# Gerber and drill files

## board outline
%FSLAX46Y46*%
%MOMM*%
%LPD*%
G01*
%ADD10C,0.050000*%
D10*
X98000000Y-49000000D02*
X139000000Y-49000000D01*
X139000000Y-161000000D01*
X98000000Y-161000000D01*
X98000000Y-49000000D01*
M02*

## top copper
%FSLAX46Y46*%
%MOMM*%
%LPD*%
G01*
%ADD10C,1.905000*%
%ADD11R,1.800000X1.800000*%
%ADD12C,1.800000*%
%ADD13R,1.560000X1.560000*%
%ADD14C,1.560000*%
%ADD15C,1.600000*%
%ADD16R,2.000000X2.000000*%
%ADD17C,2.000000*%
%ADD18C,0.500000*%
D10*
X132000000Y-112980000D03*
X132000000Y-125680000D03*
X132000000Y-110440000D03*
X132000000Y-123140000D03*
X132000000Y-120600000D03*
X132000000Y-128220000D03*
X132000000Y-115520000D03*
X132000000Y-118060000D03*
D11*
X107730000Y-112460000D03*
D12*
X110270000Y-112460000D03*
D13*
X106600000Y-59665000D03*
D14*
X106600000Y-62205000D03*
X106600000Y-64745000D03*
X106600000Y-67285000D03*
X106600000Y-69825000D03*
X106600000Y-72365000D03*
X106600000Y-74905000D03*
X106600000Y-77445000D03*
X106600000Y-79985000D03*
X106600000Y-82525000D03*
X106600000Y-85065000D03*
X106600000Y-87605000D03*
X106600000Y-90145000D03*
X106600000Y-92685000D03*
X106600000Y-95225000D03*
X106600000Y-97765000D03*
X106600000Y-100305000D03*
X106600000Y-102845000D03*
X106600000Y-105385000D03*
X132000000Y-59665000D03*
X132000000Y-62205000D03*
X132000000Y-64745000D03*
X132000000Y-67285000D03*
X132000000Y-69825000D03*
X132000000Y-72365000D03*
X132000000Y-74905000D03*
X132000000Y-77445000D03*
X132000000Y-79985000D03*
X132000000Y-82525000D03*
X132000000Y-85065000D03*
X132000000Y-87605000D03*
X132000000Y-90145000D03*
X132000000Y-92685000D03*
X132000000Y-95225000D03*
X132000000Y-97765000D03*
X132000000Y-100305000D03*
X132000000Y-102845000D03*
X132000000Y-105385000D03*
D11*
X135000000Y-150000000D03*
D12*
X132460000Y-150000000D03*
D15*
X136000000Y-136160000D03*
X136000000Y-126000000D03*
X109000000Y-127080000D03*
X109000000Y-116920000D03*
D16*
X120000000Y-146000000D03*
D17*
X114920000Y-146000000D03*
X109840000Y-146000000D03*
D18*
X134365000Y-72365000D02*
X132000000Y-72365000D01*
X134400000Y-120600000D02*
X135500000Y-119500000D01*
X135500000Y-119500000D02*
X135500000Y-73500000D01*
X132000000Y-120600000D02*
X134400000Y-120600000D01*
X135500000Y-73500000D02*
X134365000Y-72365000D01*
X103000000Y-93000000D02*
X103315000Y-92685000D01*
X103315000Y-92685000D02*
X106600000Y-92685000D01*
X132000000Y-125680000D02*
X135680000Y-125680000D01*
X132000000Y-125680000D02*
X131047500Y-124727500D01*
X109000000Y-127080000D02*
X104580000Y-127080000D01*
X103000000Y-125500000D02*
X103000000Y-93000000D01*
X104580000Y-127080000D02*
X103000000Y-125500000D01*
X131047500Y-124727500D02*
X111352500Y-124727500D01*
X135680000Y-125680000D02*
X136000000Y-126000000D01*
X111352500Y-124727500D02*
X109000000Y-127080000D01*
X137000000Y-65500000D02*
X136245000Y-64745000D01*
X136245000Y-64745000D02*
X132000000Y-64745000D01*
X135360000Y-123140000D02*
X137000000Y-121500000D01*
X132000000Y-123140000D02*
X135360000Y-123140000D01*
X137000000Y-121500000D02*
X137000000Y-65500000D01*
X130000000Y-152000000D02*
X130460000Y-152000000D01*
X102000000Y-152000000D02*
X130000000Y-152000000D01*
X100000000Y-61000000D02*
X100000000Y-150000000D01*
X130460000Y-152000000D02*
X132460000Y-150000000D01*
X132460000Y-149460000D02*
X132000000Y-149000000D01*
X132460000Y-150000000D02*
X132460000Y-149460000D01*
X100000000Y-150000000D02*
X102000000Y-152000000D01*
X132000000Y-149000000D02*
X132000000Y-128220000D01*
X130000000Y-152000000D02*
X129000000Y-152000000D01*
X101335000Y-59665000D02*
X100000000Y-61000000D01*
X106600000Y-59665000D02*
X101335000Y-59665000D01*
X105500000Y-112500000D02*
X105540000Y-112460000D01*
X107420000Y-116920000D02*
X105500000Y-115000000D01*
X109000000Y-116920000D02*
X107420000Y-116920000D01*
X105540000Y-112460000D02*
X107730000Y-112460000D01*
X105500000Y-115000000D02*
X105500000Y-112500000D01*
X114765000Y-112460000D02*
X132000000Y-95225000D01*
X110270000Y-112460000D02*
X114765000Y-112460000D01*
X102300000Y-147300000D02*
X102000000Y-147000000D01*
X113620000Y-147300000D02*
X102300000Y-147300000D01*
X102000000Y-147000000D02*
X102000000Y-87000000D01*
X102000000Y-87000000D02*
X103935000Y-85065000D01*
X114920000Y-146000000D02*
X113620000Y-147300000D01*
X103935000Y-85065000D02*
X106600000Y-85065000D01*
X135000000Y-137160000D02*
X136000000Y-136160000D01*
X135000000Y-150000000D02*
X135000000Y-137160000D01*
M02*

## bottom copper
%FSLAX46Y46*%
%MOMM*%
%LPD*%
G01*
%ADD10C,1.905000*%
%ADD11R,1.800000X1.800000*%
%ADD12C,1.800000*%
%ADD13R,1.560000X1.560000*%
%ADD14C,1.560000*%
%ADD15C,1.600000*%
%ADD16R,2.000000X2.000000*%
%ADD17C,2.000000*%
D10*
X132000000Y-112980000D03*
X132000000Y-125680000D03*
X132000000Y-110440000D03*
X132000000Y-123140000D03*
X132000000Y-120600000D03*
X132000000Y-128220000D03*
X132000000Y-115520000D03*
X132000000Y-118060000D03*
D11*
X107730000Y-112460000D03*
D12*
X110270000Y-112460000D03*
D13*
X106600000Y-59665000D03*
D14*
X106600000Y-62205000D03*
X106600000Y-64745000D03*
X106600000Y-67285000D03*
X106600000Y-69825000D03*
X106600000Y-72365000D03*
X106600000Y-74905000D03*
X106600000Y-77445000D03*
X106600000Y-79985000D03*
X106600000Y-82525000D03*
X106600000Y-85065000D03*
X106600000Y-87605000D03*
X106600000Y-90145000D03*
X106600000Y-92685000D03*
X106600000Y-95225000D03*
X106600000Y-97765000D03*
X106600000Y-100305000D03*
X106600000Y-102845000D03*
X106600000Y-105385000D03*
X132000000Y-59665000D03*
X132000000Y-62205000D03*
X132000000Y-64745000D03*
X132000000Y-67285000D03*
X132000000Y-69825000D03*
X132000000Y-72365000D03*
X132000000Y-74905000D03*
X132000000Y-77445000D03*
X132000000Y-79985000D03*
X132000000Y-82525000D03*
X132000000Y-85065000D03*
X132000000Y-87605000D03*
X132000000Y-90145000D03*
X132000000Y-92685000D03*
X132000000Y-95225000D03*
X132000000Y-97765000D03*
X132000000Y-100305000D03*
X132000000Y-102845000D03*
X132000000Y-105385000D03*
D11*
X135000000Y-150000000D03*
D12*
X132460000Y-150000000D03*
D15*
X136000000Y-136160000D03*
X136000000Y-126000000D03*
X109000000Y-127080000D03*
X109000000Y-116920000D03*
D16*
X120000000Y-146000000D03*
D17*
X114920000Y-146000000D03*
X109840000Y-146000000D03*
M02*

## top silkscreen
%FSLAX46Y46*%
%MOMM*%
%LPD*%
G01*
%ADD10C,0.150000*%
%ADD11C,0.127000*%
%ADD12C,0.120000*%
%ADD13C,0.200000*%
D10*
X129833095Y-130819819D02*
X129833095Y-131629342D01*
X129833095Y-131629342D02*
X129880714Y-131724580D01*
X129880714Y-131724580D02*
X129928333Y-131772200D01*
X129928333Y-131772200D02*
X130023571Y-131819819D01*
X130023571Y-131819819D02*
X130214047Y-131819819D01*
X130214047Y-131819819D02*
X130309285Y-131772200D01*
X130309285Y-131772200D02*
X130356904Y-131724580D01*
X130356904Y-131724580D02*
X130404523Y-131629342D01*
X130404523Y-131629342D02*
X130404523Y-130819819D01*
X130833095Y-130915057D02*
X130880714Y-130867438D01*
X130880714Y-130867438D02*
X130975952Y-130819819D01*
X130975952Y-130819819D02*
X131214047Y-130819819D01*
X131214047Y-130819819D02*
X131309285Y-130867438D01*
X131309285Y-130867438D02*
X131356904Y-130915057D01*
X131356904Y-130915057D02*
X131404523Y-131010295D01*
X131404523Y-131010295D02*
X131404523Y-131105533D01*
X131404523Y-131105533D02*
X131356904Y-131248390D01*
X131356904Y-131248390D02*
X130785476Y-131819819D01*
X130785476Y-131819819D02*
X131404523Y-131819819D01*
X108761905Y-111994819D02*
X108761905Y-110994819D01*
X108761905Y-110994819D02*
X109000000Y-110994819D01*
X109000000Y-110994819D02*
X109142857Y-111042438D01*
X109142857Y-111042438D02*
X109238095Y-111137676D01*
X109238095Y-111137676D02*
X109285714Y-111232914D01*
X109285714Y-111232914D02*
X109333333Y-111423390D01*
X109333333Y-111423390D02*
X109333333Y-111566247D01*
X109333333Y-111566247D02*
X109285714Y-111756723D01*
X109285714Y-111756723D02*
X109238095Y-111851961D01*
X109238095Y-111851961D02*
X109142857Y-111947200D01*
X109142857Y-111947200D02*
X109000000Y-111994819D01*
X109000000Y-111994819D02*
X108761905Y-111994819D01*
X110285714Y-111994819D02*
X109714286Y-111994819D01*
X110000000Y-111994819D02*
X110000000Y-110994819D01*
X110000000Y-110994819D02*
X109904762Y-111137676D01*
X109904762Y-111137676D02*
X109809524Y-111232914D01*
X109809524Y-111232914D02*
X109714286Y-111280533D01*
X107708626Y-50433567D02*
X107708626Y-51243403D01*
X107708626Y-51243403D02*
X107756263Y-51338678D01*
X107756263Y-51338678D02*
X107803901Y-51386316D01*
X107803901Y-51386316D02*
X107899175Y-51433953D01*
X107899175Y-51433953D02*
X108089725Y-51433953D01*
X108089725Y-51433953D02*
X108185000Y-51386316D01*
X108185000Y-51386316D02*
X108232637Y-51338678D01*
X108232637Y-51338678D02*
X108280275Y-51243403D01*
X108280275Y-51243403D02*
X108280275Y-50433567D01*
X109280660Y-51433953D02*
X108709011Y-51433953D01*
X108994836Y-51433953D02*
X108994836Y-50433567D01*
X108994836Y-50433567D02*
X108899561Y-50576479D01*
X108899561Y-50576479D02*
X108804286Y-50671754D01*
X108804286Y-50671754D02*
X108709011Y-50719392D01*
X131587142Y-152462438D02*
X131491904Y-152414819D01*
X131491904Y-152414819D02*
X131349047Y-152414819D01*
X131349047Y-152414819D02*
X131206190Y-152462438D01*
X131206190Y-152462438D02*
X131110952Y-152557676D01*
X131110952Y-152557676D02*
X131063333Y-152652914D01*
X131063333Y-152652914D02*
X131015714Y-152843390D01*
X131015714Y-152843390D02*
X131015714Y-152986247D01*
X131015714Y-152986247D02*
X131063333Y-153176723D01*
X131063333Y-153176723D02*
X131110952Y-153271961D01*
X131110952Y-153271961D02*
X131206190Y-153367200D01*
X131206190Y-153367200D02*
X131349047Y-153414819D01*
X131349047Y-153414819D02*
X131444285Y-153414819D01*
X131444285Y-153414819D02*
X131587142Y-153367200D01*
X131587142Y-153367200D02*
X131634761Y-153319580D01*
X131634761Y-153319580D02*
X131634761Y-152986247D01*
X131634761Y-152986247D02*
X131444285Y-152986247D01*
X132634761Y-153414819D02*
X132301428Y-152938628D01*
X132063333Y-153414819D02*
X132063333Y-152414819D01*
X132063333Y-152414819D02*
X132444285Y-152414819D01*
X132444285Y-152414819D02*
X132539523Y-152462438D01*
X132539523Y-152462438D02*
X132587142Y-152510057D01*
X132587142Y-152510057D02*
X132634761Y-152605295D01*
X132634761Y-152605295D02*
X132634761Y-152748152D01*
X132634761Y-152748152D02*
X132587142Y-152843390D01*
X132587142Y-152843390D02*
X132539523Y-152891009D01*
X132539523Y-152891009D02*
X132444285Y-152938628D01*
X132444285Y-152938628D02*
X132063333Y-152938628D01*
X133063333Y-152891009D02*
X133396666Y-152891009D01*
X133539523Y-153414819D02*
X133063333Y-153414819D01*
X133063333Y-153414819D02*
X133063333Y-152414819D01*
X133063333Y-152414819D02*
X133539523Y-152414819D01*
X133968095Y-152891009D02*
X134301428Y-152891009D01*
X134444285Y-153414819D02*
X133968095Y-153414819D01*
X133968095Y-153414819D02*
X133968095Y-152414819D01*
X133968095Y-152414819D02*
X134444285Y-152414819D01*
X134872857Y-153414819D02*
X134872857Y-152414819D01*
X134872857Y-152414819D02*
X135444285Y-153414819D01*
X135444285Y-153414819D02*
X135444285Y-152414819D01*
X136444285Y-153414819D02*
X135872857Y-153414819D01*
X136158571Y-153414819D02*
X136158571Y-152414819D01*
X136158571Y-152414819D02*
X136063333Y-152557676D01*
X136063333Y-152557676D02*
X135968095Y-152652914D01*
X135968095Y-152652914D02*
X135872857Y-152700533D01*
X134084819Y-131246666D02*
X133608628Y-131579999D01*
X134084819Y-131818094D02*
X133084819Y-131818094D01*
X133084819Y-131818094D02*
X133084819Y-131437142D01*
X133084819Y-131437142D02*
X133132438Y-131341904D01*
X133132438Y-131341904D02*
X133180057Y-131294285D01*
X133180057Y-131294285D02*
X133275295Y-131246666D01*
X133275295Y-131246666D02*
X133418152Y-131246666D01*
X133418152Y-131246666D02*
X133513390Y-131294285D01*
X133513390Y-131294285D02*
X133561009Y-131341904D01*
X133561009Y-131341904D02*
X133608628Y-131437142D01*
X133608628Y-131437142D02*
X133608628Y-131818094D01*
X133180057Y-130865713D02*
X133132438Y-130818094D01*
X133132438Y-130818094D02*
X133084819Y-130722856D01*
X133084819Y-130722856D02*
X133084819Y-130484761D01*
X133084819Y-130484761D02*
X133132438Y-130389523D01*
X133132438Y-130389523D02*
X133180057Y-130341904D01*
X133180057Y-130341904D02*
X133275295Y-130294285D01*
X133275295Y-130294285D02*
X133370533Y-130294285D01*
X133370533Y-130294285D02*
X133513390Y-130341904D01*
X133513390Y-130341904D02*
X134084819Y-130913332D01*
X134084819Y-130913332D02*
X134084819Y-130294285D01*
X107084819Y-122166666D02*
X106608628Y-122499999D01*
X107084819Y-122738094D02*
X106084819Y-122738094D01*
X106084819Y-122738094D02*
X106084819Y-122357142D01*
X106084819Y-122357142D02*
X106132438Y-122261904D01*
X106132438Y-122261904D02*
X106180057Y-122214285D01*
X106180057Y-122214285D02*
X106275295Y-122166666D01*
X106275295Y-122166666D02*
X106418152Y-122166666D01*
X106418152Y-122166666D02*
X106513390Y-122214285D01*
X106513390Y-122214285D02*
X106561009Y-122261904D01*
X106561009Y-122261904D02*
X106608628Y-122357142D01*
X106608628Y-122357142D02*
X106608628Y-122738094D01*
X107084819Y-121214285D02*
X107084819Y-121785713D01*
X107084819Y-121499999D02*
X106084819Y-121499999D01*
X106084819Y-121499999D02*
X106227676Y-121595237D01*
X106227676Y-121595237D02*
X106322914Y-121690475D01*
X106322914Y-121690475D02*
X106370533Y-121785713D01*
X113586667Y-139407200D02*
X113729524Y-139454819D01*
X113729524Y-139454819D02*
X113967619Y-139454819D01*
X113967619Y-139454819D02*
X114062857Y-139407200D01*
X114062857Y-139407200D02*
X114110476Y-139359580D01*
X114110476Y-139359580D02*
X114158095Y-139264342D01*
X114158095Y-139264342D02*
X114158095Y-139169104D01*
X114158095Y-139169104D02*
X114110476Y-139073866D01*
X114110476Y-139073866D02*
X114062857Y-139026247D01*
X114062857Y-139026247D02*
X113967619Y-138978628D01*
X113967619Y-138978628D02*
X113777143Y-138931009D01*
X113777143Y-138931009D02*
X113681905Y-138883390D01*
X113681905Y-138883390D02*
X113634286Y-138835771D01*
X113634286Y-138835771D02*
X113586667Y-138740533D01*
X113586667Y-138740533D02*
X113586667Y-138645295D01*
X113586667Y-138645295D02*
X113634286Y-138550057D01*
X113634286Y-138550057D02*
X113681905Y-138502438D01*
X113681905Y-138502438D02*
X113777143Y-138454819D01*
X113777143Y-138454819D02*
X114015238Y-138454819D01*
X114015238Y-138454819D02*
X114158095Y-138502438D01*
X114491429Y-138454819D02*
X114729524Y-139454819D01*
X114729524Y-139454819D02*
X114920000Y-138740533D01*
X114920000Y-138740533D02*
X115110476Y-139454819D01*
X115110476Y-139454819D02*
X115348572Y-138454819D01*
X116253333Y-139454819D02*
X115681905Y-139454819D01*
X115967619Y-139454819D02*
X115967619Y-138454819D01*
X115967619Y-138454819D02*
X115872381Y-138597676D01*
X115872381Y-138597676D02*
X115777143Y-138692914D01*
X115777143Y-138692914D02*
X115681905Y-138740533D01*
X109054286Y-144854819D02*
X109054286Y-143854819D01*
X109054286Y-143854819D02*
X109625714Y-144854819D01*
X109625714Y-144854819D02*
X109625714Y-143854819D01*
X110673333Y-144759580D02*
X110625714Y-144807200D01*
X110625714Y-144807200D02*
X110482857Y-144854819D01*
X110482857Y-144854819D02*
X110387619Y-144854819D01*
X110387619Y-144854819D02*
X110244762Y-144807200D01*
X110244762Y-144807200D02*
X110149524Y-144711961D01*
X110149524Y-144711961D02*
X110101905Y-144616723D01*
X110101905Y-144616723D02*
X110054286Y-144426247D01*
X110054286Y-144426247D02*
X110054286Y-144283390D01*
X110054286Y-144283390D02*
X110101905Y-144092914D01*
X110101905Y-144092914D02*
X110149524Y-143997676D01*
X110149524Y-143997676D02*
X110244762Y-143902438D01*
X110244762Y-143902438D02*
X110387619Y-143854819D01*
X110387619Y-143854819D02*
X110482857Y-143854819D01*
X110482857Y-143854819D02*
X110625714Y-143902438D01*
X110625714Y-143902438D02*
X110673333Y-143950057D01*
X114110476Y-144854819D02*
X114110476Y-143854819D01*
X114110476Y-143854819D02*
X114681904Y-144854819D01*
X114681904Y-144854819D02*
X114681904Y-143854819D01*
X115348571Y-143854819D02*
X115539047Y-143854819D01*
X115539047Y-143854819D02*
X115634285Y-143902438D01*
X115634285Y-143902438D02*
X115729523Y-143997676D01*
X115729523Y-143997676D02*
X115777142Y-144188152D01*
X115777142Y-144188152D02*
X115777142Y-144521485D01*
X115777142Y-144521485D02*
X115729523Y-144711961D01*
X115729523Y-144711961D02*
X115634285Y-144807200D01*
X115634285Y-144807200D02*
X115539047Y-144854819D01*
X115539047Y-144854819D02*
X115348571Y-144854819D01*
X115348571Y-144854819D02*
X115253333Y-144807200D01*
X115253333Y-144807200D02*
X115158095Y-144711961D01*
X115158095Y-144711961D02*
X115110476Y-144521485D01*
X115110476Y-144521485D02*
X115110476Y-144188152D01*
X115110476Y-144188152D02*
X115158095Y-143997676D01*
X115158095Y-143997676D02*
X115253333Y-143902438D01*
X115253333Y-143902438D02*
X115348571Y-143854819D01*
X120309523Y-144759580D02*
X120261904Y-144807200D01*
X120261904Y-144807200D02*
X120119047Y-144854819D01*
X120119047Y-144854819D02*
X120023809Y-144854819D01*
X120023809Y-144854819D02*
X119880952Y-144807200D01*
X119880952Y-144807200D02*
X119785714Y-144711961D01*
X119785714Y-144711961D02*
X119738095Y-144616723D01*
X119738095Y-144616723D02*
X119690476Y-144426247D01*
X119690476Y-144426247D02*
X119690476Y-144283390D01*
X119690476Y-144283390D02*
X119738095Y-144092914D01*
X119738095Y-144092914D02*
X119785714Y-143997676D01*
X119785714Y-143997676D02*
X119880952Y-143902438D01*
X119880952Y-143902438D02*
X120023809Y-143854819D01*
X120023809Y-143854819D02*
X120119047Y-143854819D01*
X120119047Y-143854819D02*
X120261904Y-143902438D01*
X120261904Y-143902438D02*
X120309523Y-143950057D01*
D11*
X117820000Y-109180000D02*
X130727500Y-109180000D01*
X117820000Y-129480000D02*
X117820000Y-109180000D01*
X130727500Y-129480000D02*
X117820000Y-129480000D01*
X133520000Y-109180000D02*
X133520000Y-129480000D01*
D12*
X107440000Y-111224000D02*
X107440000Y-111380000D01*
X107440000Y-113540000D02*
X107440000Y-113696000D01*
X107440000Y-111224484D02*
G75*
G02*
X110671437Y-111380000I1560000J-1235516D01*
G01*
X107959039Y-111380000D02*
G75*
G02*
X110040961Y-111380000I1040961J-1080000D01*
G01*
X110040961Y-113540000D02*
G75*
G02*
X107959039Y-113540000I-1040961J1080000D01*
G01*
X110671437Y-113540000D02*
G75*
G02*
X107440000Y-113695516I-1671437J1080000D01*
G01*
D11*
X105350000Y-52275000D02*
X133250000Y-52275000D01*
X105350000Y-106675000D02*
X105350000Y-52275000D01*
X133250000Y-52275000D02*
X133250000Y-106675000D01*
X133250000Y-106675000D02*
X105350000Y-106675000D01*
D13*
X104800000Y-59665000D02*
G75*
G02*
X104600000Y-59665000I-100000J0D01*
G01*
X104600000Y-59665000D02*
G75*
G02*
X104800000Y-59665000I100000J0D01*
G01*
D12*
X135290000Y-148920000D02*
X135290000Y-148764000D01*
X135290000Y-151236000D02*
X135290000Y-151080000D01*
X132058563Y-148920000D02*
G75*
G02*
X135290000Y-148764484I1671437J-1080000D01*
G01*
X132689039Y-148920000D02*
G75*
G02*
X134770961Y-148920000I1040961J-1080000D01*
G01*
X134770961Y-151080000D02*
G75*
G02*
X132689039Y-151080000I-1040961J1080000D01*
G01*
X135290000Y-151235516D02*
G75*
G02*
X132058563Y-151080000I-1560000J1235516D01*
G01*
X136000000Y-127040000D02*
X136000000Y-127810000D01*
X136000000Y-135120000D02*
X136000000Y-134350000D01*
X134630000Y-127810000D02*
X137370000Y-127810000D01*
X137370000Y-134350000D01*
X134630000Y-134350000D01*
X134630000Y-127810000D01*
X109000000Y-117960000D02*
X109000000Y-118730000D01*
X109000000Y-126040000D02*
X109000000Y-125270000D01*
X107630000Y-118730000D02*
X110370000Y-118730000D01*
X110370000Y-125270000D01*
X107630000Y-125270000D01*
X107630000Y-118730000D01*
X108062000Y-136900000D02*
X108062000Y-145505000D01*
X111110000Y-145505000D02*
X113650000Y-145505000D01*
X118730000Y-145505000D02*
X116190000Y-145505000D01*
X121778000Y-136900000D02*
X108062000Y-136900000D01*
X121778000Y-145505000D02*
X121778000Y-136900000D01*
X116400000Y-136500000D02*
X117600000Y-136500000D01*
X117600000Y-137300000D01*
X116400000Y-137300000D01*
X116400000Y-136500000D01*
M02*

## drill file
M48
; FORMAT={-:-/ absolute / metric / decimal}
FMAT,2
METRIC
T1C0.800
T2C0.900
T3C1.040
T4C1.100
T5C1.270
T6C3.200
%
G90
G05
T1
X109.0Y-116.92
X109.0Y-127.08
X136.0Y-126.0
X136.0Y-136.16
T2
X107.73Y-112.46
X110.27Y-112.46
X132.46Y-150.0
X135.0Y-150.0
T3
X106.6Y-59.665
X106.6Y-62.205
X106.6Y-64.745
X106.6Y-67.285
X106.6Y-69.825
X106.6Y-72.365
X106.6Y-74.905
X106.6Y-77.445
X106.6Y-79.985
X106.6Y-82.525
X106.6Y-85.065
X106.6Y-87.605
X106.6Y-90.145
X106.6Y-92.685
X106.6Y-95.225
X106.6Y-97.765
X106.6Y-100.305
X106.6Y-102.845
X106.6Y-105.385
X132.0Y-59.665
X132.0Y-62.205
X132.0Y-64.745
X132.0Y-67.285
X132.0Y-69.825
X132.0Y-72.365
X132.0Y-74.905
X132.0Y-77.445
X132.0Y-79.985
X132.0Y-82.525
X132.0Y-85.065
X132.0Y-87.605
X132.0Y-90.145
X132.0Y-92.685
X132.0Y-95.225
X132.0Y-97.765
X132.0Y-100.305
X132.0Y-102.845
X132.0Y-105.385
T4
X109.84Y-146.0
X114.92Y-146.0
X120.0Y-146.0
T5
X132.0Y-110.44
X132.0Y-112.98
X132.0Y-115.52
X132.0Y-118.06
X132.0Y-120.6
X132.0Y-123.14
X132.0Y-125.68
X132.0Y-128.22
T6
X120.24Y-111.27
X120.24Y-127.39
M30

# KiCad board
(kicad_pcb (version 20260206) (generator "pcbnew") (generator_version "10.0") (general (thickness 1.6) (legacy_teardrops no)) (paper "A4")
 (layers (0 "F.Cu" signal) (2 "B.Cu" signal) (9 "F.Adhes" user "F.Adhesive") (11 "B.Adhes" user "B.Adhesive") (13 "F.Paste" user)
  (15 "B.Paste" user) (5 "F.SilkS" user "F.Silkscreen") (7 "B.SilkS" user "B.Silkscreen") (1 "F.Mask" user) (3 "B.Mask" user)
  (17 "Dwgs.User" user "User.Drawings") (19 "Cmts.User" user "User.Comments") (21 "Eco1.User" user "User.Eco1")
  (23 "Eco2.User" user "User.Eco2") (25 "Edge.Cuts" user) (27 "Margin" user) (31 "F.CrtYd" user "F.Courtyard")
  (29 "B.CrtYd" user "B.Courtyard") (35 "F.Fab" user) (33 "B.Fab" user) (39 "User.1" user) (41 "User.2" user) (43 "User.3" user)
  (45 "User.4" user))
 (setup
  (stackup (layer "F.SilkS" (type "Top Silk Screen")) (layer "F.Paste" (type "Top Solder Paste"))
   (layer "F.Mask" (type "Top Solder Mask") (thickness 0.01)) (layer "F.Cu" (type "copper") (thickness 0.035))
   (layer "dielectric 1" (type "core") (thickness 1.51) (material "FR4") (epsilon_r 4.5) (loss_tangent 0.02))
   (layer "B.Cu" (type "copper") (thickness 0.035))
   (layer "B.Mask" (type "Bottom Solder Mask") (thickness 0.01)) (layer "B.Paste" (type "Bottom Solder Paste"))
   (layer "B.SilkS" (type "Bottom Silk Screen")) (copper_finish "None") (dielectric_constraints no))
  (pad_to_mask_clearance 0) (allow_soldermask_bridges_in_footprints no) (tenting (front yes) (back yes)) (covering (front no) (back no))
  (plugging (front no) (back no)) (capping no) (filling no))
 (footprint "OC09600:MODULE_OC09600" (layer "F.Cu") (at 125.67 119.33 180)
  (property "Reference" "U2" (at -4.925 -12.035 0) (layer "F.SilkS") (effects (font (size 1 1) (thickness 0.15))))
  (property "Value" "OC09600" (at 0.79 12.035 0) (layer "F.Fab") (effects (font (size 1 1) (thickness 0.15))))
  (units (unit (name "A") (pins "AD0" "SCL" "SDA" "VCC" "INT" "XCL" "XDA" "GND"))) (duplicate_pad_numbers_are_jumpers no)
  (fp_line (start 7.85 10.15) (end -5.0575 10.15) (stroke (width 0.127) (type solid)) (layer "F.SilkS"))
  (fp_line (start 7.85 -10.15) (end 7.85 10.15) (stroke (width 0.127) (type solid)) (layer "F.SilkS"))
  (fp_line (start -5.0575 -10.15) (end 7.85 -10.15) (stroke (width 0.127) (type solid)) (layer "F.SilkS"))
  (fp_line (start -7.85 10.15) (end -7.85 -10.15) (stroke (width 0.127) (type solid)) (layer "F.SilkS"))
  (pad "" np_thru_hole circle (at 5.43 -8.06 180) (size 3.2 3.2) (drill 3.2) (layers "*.Cu" "*.Mask"))
  (pad "" np_thru_hole circle (at 5.43 8.06 180) (size 3.2 3.2) (drill 3.2) (layers "*.Cu" "*.Mask"))
  (pad "AD0" thru_hole circle (at -6.33 6.35 180) (size 1.905 1.905) (drill 1.27) (layers "*.Cu" "*.Mask") (remove_unused_layers no)
   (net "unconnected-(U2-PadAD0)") (solder_mask_margin 0.102))
  (pad "GND" thru_hole circle (at -6.33 -6.35 180) (size 1.905 1.905) (drill 1.27) (layers "*.Cu" "*.Mask") (remove_unused_layers no)
   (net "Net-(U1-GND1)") (solder_mask_margin 0.102))
  (pad "INT" thru_hole circle (at -6.33 8.89 180) (size 1.905 1.905) (drill 1.27) (layers "*.Cu" "*.Mask") (remove_unused_layers no)
   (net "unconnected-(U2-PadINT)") (solder_mask_margin 0.102))
  (pad "SCL" thru_hole circle (at -6.33 -3.81 180) (size 1.905 1.905) (drill 1.27) (layers "*.Cu" "*.Mask") (remove_unused_layers no)
   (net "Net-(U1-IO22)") (solder_mask_margin 0.102))
  (pad "SDA" thru_hole circle (at -6.33 -1.27 180) (size 1.905 1.905) (drill 1.27) (layers "*.Cu" "*.Mask") (remove_unused_layers no)
   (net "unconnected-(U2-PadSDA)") (solder_mask_margin 0.102))
  (pad "VCC" thru_hole circle (at -6.33 -8.89 180) (size 1.905 1.905) (drill 1.27) (layers "*.Cu" "*.Mask") (remove_unused_layers no)
   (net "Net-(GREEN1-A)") (solder_mask_margin 0.102))
  (pad "XCL" thru_hole circle (at -6.33 3.81 180) (size 1.905 1.905) (drill 1.27) (layers "*.Cu" "*.Mask") (remove_unused_layers no)
   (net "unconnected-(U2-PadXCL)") (solder_mask_margin 0.102))
  (pad "XDA" thru_hole circle (at -6.33 1.27 180) (size 1.905 1.905) (drill 1.27) (layers "*.Cu" "*.Mask") (remove_unused_layers no)
   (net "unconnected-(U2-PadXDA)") (solder_mask_margin 0.102)))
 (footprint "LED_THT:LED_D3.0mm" (layer "F.Cu") (at 107.73 112.46)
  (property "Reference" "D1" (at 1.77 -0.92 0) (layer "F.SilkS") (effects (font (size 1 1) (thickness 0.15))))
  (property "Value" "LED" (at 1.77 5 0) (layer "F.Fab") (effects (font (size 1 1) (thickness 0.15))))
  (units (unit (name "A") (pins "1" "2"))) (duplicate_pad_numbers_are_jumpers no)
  (fp_line (start -0.29 -1.236) (end -0.29 -1.08) (stroke (width 0.12) (type solid)) (layer "F.SilkS"))
  (fp_line (start -0.29 1.08) (end -0.29 1.236) (stroke (width 0.12) (type solid)) (layer "F.SilkS"))
  (fp_arc (start -0.29 -1.235516) (mid 1.36566 -1.987699) (end 2.941437 -1.08) (stroke (width 0.12) (type solid)) (layer "F.SilkS"))
  (fp_arc (start 0.229039 -1.08) (mid 1.27 -1.5) (end 2.310961 -1.08) (stroke (width 0.12) (type solid)) (layer "F.SilkS"))
  (fp_arc (start 2.310961 1.08) (mid 1.27 1.5) (end 0.229039 1.08) (stroke (width 0.12) (type solid)) (layer "F.SilkS"))
  (fp_arc (start 2.941437 1.08) (mid 1.36566 1.987699) (end -0.29 1.235516) (stroke (width 0.12) (type solid)) (layer "F.SilkS"))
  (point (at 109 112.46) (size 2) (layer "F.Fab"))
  (pad "1" thru_hole rect (at 0 0) (size 1.8 1.8) (drill 0.9) (layers "*.Cu" "*.Mask") (remove_unused_layers no) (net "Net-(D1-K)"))
  (pad "2" thru_hole circle (at 2.54 0) (size 1.8 1.8) (drill 0.9) (layers "*.Cu" "*.Mask") (remove_unused_layers no) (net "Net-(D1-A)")))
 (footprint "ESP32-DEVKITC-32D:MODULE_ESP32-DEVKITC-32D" (layer "F.Cu") (at 119.3 79.425)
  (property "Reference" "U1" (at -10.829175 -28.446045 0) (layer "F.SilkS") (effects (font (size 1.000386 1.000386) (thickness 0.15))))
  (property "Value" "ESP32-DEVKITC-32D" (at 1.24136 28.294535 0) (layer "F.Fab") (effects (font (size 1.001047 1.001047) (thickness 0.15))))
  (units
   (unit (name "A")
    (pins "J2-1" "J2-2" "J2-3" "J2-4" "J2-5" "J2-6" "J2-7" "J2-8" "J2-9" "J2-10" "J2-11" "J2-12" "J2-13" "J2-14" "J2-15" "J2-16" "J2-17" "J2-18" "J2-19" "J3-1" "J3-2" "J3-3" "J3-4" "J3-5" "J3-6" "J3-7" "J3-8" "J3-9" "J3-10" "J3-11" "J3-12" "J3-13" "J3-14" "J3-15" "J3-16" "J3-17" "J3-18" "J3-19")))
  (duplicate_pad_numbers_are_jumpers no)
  (fp_line (start -13.95 -27.15) (end 13.95 -27.15) (stroke (width 0.127) (type solid)) (layer "F.SilkS"))
  (fp_line (start -13.95 27.25) (end -13.95 -27.15) (stroke (width 0.127) (type solid)) (layer "F.SilkS"))
  (fp_line (start 13.95 -27.15) (end 13.95 27.25) (stroke (width 0.127) (type solid)) (layer "F.SilkS"))
  (fp_line (start 13.95 27.25) (end -13.95 27.25) (stroke (width 0.127) (type solid)) (layer "F.SilkS"))
  (fp_circle (center -14.6 -19.76) (end -14.5 -19.76) (stroke (width 0.2) (type solid)) (fill no) (layer "F.SilkS"))
  (pad "J2-1" thru_hole rect (at -12.7 -19.76) (size 1.56 1.56) (drill 1.04) (layers "*.Cu" "*.Mask") (remove_unused_layers no)
   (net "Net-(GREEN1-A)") (solder_mask_margin 0.102))
  (pad "J2-2" thru_hole circle (at -12.7 -17.22) (size 1.56 1.56) (drill 1.04) (layers "*.Cu" "*.Mask") (remove_unused_layers no)
   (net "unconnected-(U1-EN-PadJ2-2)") (solder_mask_margin 0.102))
  (pad "J2-3" thru_hole circle (at -12.7 -14.68) (size 1.56 1.56) (drill 1.04) (layers "*.Cu" "*.Mask") (remove_unused_layers no)
   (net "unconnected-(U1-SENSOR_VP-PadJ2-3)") (solder_mask_margin 0.102))
  (pad "J2-4" thru_hole circle (at -12.7 -12.14) (size 1.56 1.56) (drill 1.04) (layers "*.Cu" "*.Mask") (remove_unused_layers no)
   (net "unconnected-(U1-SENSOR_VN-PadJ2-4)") (solder_mask_margin 0.102))
  (pad "J2-5" thru_hole circle (at -12.7 -9.6) (size 1.56 1.56) (drill 1.04) (layers "*.Cu" "*.Mask") (remove_unused_layers no)
   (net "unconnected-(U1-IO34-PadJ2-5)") (solder_mask_margin 0.102))
  (pad "J2-6" thru_hole circle (at -12.7 -7.06) (size 1.56 1.56) (drill 1.04) (layers "*.Cu" "*.Mask") (remove_unused_layers no)
   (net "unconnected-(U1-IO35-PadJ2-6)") (solder_mask_margin 0.102))
  (pad "J2-7" thru_hole circle (at -12.7 -4.52) (size 1.56 1.56) (drill 1.04) (layers "*.Cu" "*.Mask") (remove_unused_layers no)
   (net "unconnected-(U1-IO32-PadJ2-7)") (solder_mask_margin 0.102))
  (pad "J2-8" thru_hole circle (at -12.7 -1.98) (size 1.56 1.56) (drill 1.04) (layers "*.Cu" "*.Mask") (remove_unused_layers no)
   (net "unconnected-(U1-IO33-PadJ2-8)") (solder_mask_margin 0.102))
  (pad "J2-9" thru_hole circle (at -12.7 0.56) (size 1.56 1.56) (drill 1.04) (layers "*.Cu" "*.Mask") (remove_unused_layers no)
   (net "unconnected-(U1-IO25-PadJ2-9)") (solder_mask_margin 0.102))
  (pad "J2-10" thru_hole circle (at -12.7 3.1) (size 1.56 1.56) (drill 1.04) (layers "*.Cu" "*.Mask") (remove_unused_layers no)
   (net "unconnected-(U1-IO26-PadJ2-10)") (solder_mask_margin 0.102))
  (pad "J2-11" thru_hole circle (at -12.7 5.64) (size 1.56 1.56) (drill 1.04) (layers "*.Cu" "*.Mask") (remove_unused_layers no)
   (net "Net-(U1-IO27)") (solder_mask_margin 0.102))
  (pad "J2-12" thru_hole circle (at -12.7 8.18) (size 1.56 1.56) (drill 1.04) (layers "*.Cu" "*.Mask") (remove_unused_layers no)
   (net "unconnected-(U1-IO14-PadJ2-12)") (solder_mask_margin 0.102))
  (pad "J2-13" thru_hole circle (at -12.7 10.72) (size 1.56 1.56) (drill 1.04) (layers "*.Cu" "*.Mask") (remove_unused_layers no)
   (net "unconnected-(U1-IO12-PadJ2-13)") (solder_mask_margin 0.102))
  (pad "J2-14" thru_hole circle (at -12.7 13.26) (size 1.56 1.56) (drill 1.04) (layers "*.Cu" "*.Mask") (remove_unused_layers no)
   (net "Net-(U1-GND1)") (solder_mask_margin 0.102))
  (pad "J2-15" thru_hole circle (at -12.7 15.8) (size 1.56 1.56) (drill 1.04) (layers "*.Cu" "*.Mask") (remove_unused_layers no)
   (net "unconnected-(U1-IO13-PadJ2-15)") (solder_mask_margin 0.102))
  (pad "J2-16" thru_hole circle (at -12.7 18.34) (size 1.56 1.56) (drill 1.04) (layers "*.Cu" "*.Mask") (remove_unused_layers no)
   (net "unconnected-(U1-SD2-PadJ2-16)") (solder_mask_margin 0.102))
  (pad "J2-17" thru_hole circle (at -12.7 20.88) (size 1.56 1.56) (drill 1.04) (layers "*.Cu" "*.Mask") (remove_unused_layers no)
   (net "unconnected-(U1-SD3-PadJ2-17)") (solder_mask_margin 0.102))
  (pad "J2-18" thru_hole circle (at -12.7 23.42) (size 1.56 1.56) (drill 1.04) (layers "*.Cu" "*.Mask") (remove_unused_layers no)
   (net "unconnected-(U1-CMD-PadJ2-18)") (solder_mask_margin 0.102))
  (pad "J2-19" thru_hole circle (at -12.7 25.96) (size 1.56 1.56) (drill 1.04) (layers "*.Cu" "*.Mask") (remove_unused_layers no)
   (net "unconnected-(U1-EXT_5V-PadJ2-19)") (solder_mask_margin 0.102))
  (pad "J3-1" thru_hole circle (at 12.7 -19.76) (size 1.56 1.56) (drill 1.04) (layers "*.Cu" "*.Mask") (remove_unused_layers no)
   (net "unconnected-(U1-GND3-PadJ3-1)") (solder_mask_margin 0.102))
  (pad "J3-2" thru_hole circle (at 12.7 -17.22) (size 1.56 1.56) (drill 1.04) (layers "*.Cu" "*.Mask") (remove_unused_layers no)
   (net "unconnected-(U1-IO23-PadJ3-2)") (solder_mask_margin 0.102))
  (pad "J3-3" thru_hole circle (at 12.7 -14.68) (size 1.56 1.56) (drill 1.04) (layers "*.Cu" "*.Mask") (remove_unused_layers no)
   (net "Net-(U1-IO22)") (solder_mask_margin 0.102))
  (pad "J3-4" thru_hole circle (at 12.7 -12.14) (size 1.56 1.56) (drill 1.04) (layers "*.Cu" "*.Mask") (remove_unused_layers no)
   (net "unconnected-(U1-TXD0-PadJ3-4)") (solder_mask_margin 0.102))
  (pad "J3-5" thru_hole circle (at 12.7 -9.6) (size 1.56 1.56) (drill 1.04) (layers "*.Cu" "*.Mask") (remove_unused_layers no)
   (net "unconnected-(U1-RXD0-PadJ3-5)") (solder_mask_margin 0.102))
  (pad "J3-6" thru_hole circle (at 12.7 -7.06) (size 1.56 1.56) (drill 1.04) (layers "*.Cu" "*.Mask") (remove_unused_layers no)
   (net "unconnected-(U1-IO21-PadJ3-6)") (solder_mask_margin 0.102))
  (pad "J3-7" thru_hole circle (at 12.7 -4.52) (size 1.56 1.56) (drill 1.04) (layers "*.Cu" "*.Mask") (remove_unused_layers no)
   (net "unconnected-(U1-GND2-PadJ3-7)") (solder_mask_margin 0.102))
  (pad "J3-8" thru_hole circle (at 12.7 -1.98) (size 1.56 1.56) (drill 1.04) (layers "*.Cu" "*.Mask") (remove_unused_layers no)
   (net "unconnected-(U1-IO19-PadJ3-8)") (solder_mask_margin 0.102))
  (pad "J3-9" thru_hole circle (at 12.7 0.56) (size 1.56 1.56) (drill 1.04) (layers "*.Cu" "*.Mask") (remove_unused_layers no)
   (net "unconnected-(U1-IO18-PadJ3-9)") (solder_mask_margin 0.102))
  (pad "J3-10" thru_hole circle (at 12.7 3.1) (size 1.56 1.56) (drill 1.04) (layers "*.Cu" "*.Mask") (remove_unused_layers no)
   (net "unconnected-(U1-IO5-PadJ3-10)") (solder_mask_margin 0.102))
  (pad "J3-11" thru_hole circle (at 12.7 5.64) (size 1.56 1.56) (drill 1.04) (layers "*.Cu" "*.Mask") (remove_unused_layers no)
   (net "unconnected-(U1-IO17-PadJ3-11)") (solder_mask_margin 0.102))
  (pad "J3-12" thru_hole circle (at 12.7 8.18) (size 1.56 1.56) (drill 1.04) (layers "*.Cu" "*.Mask") (remove_unused_layers no)
   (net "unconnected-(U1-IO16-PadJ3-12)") (solder_mask_margin 0.102))
  (pad "J3-13" thru_hole circle (at 12.7 10.72) (size 1.56 1.56) (drill 1.04) (layers "*.Cu" "*.Mask") (remove_unused_layers no)
   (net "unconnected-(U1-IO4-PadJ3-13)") (solder_mask_margin 0.102))
  (pad "J3-14" thru_hole circle (at 12.7 13.26) (size 1.56 1.56) (drill 1.04) (layers "*.Cu" "*.Mask") (remove_unused_layers no)
   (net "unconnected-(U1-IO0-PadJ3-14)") (solder_mask_margin 0.102))
  (pad "J3-15" thru_hole circle (at 12.7 15.8) (size 1.56 1.56) (drill 1.04) (layers "*.Cu" "*.Mask") (remove_unused_layers no)
   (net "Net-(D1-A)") (solder_mask_margin 0.102))
  (pad "J3-16" thru_hole circle (at 12.7 18.34) (size 1.56 1.56) (drill 1.04) (layers "*.Cu" "*.Mask") (remove_unused_layers no)
   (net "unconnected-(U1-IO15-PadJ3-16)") (solder_mask_margin 0.102))
  (pad "J3-17" thru_hole circle (at 12.7 20.88) (size 1.56 1.56) (drill 1.04) (layers "*.Cu" "*.Mask") (remove_unused_layers no)
   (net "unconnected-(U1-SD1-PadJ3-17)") (solder_mask_margin 0.102))
  (pad "J3-18" thru_hole circle (at 12.7 23.42) (size 1.56 1.56) (drill 1.04) (layers "*.Cu" "*.Mask") (remove_unused_layers no)
   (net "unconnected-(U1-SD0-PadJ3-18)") (solder_mask_margin 0.102))
  (pad "J3-19" thru_hole circle (at 12.7 25.96) (size 1.56 1.56) (drill 1.04) (layers "*.Cu" "*.Mask") (remove_unused_layers no)
   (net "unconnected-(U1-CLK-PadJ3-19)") (solder_mask_margin 0.102)))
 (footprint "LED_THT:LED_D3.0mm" (layer "F.Cu") (at 135 150 180)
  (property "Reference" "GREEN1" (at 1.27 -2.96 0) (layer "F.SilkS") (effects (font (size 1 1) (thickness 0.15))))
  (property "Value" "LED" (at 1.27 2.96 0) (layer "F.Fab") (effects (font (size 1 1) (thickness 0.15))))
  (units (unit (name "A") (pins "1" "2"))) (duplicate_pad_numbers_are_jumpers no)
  (fp_line (start -0.29 1.08) (end -0.29 1.236) (stroke (width 0.12) (type solid)) (layer "F.SilkS"))
  (fp_line (start -0.29 -1.236) (end -0.29 -1.08) (stroke (width 0.12) (type solid)) (layer "F.SilkS"))
  (fp_arc (start 2.941437 1.08) (mid 1.36566 1.987699) (end -0.29 1.235516) (stroke (width 0.12) (type solid)) (layer "F.SilkS"))
  (fp_arc (start 2.310961 1.08) (mid 1.27 1.5) (end 0.229039 1.08) (stroke (width 0.12) (type solid)) (layer "F.SilkS"))
  (fp_arc (start 0.229039 -1.08) (mid 1.27 -1.5) (end 2.310961 -1.08) (stroke (width 0.12) (type solid)) (layer "F.SilkS"))
  (fp_arc (start -0.29 -1.235516) (mid 1.36566 -1.987699) (end 2.941437 -1.08) (stroke (width 0.12) (type solid)) (layer "F.SilkS"))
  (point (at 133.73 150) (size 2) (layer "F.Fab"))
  (pad "1" thru_hole rect (at 0 0 180) (size 1.8 1.8) (drill 0.9) (layers "*.Cu" "*.Mask") (remove_unused_layers no) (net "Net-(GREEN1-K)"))
  (pad "2" thru_hole circle (at 2.54 0 180) (size 1.8 1.8) (drill 0.9) (layers "*.Cu" "*.Mask") (remove_unused_layers no)
   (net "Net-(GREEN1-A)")))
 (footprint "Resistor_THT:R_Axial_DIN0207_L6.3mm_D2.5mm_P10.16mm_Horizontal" (layer "F.Cu") (at 136 136.16 90)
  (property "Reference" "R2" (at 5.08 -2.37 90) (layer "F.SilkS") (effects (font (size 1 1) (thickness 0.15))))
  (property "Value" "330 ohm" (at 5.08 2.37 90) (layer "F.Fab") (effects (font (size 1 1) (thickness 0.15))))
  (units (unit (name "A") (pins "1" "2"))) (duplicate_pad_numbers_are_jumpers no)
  (fp_line (start 9.12 0) (end 8.35 0) (stroke (width 0.12) (type solid)) (layer "F.SilkS"))
  (fp_line (start 1.04 0) (end 1.81 0) (stroke (width 0.12) (type solid)) (layer "F.SilkS"))
  (fp_rect (start 1.81 -1.37) (end 8.35 1.37) (stroke (width 0.12) (type solid)) (fill no) (layer "F.SilkS"))
  (pad "1" thru_hole circle (at 0 0 90) (size 1.6 1.6) (drill 0.8) (layers "*.Cu" "*.Mask") (remove_unused_layers no) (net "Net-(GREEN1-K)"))
  (pad "2" thru_hole circle (at 10.16 0 90) (size 1.6 1.6) (drill 0.8) (layers "*.Cu" "*.Mask") (remove_unused_layers no)
   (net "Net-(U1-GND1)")))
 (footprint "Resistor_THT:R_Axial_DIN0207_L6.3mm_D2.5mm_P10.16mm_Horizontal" (layer "F.Cu") (at 109 127.08 90)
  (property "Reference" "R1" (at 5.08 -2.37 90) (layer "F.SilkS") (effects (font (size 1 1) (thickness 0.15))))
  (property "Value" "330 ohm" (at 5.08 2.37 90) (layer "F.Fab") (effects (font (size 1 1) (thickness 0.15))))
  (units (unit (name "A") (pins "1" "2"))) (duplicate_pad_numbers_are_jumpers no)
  (fp_line (start 9.12 0) (end 8.35 0) (stroke (width 0.12) (type solid)) (layer "F.SilkS"))
  (fp_line (start 1.04 0) (end 1.81 0) (stroke (width 0.12) (type solid)) (layer "F.SilkS"))
  (fp_rect (start 1.81 -1.37) (end 8.35 1.37) (stroke (width 0.12) (type solid)) (fill no) (layer "F.SilkS"))
  (pad "1" thru_hole circle (at 0 0 90) (size 1.6 1.6) (drill 0.8) (layers "*.Cu" "*.Mask") (remove_unused_layers no) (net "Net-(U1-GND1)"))
  (pad "2" thru_hole circle (at 10.16 0 90) (size 1.6 1.6) (drill 0.8) (layers "*.Cu" "*.Mask") (remove_unused_layers no) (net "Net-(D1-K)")))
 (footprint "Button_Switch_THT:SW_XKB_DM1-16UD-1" (layer "F.Cu") (at 120 146)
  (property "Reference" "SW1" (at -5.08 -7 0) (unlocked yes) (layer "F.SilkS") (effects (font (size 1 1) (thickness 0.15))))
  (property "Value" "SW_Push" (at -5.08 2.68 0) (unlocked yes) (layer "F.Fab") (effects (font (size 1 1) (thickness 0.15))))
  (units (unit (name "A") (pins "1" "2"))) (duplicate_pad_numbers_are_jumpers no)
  (fp_line (start -11.938 -9.1) (end -11.938 -0.495) (stroke (width 0.12) (type solid)) (layer "F.SilkS"))
  (fp_line (start -8.89 -0.495) (end -6.35 -0.495) (stroke (width 0.12) (type solid)) (layer "F.SilkS"))
  (fp_line (start -1.27 -0.495) (end -3.81 -0.495) (stroke (width 0.12) (type solid)) (layer "F.SilkS"))
  (fp_line (start 1.778 -9.1) (end -11.938 -9.1) (stroke (width 0.12) (type solid)) (layer "F.SilkS"))
  (fp_line (start 1.778 -0.495) (end 1.778 -9.1) (stroke (width 0.12) (type solid)) (layer "F.SilkS"))
  (fp_rect (start -3.6 -9.5) (end -2.4 -8.7) (stroke (width 0.12) (type solid)) (fill no) (layer "F.SilkS"))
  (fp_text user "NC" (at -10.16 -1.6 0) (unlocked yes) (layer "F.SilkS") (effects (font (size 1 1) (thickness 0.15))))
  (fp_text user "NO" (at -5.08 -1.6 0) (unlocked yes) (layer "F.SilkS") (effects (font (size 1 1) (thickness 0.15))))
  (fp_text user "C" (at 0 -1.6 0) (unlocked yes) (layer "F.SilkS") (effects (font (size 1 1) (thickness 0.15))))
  (pad "1" thru_hole rect (at 0 0) (size 2 2) (drill 1.1) (layers "*.Cu" "*.Mask") (remove_unused_layers no) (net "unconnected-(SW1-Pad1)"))
  (pad "2" thru_hole circle (at -5.08 0) (size 2 2) (drill 1.1) (layers "*.Cu" "*.Mask") (remove_unused_layers no) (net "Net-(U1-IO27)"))
  (pad "3" thru_hole circle (at -10.16 0) (size 2 2) (drill 1.1) (layers "*.Cu" "*.Mask") (remove_unused_layers no)))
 (gr_rect (start 98 49) (end 139 161) (stroke (width 0.05) (type default)) (fill no) (layer "Edge.Cuts"))
 (segment (start 134.365 72.365) (end 132 72.365) (width 0.5) (layer "F.Cu") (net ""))
 (segment (start 134.4 120.6) (end 135.5 119.5) (width 0.5) (layer "F.Cu") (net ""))
 (segment (start 135.5 119.5) (end 135.5 73.5) (width 0.5) (layer "F.Cu") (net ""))
 (segment (start 132 120.6) (end 134.4 120.6) (width 0.5) (layer "F.Cu") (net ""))
 (segment (start 135.5 73.5) (end 134.365 72.365) (width 0.5) (layer "F.Cu") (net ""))
 (segment (start 103 93) (end 103.315 92.685) (width 0.5) (layer "F.Cu") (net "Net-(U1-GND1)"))
 (segment (start 103.315 92.685) (end 106.6 92.685) (width 0.5) (layer "F.Cu") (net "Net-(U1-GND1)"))
 (segment (start 132 125.68) (end 135.68 125.68) (width 0.5) (layer "F.Cu") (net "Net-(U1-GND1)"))
 (segment (start 132 125.68) (end 131.0475 124.7275) (width 0.5) (layer "F.Cu") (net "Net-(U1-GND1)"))
 (segment (start 109 127.08) (end 104.58 127.08) (width 0.5) (layer "F.Cu") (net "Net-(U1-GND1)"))
 (segment (start 103 125.5) (end 103 93) (width 0.5) (layer "F.Cu") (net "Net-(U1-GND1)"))
 (segment (start 104.58 127.08) (end 103 125.5) (width 0.5) (layer "F.Cu") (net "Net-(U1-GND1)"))
 (segment (start 131.0475 124.7275) (end 111.3525 124.7275) (width 0.5) (layer "F.Cu") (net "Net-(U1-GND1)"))
 (segment (start 135.68 125.68) (end 136 126) (width 0.5) (layer "F.Cu") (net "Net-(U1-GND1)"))
 (segment (start 111.3525 124.7275) (end 109 127.08) (width 0.5) (layer "F.Cu") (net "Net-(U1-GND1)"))
 (segment (start 137 65.5) (end 136.245 64.745) (width 0.5) (layer "F.Cu") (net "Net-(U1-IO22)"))
 (segment (start 136.245 64.745) (end 132 64.745) (width 0.5) (layer "F.Cu") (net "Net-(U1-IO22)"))
 (segment (start 135.36 123.14) (end 137 121.5) (width 0.5) (layer "F.Cu") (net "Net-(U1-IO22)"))
 (segment (start 132 123.14) (end 135.36 123.14) (width 0.5) (layer "F.Cu") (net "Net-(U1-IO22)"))
 (segment (start 137 121.5) (end 137 65.5) (width 0.5) (layer "F.Cu") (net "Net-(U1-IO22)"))
 (segment (start 130 152) (end 130.46 152) (width 0.5) (layer "F.Cu") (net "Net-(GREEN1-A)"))
 (segment (start 102 152) (end 130 152) (width 0.5) (layer "F.Cu") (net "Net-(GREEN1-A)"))
 (segment (start 100 61) (end 100 150) (width 0.5) (layer "F.Cu") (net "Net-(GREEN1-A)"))
 (segment (start 130.46 152) (end 132.46 150) (width 0.5) (layer "F.Cu") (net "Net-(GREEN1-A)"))
 (segment (start 132.46 149.46) (end 132 149) (width 0.5) (layer "F.Cu") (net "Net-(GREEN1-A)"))
 (segment (start 132.46 150) (end 132.46 149.46) (width 0.5) (layer "F.Cu") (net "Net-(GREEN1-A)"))
 (segment (start 100 150) (end 102 152) (width 0.5) (layer "F.Cu") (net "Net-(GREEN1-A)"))
 (segment (start 132 149) (end 132 128.22) (width 0.5) (layer "F.Cu") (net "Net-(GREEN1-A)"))
 (segment (start 130 152) (end 129 152) (width 0.5) (layer "F.Cu") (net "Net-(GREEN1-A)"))
 (segment (start 101.335 59.665) (end 100 61) (width 0.5) (layer "F.Cu") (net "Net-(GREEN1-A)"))
 (segment (start 106.6 59.665) (end 101.335 59.665) (width 0.5) (layer "F.Cu") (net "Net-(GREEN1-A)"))
 (segment (start 105.5 112.5) (end 105.54 112.46) (width 0.5) (layer "F.Cu") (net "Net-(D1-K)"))
 (segment (start 107.42 116.92) (end 105.5 115) (width 0.5) (layer "F.Cu") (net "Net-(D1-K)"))
 (segment (start 109 116.92) (end 107.42 116.92) (width 0.5) (layer "F.Cu") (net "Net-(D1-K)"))
 (segment (start 105.54 112.46) (end 107.73 112.46) (width 0.5) (layer "F.Cu") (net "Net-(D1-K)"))
 (segment (start 105.5 115) (end 105.5 112.5) (width 0.5) (layer "F.Cu") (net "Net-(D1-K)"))
 (segment (start 114.765 112.46) (end 132 95.225) (width 0.5) (layer "F.Cu") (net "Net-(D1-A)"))
 (segment (start 110.27 112.46) (end 114.765 112.46) (width 0.5) (layer "F.Cu") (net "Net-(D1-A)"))
 (segment (start 102.3 147.3) (end 102 147) (width 0.5) (layer "F.Cu") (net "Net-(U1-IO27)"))
 (segment (start 113.62 147.3) (end 102.3 147.3) (width 0.5) (layer "F.Cu") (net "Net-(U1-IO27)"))
 (segment (start 102 147) (end 102 87) (width 0.5) (layer "F.Cu") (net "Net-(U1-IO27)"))
 (segment (start 102 87) (end 103.935 85.065) (width 0.5) (layer "F.Cu") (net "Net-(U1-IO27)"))
 (segment (start 114.92 146) (end 113.62 147.3) (width 0.5) (layer "F.Cu") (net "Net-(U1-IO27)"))
 (segment (start 103.935 85.065) (end 106.6 85.065) (width 0.5) (layer "F.Cu") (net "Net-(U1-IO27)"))
 (segment (start 135 137.16) (end 136 136.16) (width 0.5) (layer "F.Cu") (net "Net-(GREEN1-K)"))
 (segment (start 135 150) (end 135 137.16) (width 0.5) (layer "F.Cu") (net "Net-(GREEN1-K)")))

